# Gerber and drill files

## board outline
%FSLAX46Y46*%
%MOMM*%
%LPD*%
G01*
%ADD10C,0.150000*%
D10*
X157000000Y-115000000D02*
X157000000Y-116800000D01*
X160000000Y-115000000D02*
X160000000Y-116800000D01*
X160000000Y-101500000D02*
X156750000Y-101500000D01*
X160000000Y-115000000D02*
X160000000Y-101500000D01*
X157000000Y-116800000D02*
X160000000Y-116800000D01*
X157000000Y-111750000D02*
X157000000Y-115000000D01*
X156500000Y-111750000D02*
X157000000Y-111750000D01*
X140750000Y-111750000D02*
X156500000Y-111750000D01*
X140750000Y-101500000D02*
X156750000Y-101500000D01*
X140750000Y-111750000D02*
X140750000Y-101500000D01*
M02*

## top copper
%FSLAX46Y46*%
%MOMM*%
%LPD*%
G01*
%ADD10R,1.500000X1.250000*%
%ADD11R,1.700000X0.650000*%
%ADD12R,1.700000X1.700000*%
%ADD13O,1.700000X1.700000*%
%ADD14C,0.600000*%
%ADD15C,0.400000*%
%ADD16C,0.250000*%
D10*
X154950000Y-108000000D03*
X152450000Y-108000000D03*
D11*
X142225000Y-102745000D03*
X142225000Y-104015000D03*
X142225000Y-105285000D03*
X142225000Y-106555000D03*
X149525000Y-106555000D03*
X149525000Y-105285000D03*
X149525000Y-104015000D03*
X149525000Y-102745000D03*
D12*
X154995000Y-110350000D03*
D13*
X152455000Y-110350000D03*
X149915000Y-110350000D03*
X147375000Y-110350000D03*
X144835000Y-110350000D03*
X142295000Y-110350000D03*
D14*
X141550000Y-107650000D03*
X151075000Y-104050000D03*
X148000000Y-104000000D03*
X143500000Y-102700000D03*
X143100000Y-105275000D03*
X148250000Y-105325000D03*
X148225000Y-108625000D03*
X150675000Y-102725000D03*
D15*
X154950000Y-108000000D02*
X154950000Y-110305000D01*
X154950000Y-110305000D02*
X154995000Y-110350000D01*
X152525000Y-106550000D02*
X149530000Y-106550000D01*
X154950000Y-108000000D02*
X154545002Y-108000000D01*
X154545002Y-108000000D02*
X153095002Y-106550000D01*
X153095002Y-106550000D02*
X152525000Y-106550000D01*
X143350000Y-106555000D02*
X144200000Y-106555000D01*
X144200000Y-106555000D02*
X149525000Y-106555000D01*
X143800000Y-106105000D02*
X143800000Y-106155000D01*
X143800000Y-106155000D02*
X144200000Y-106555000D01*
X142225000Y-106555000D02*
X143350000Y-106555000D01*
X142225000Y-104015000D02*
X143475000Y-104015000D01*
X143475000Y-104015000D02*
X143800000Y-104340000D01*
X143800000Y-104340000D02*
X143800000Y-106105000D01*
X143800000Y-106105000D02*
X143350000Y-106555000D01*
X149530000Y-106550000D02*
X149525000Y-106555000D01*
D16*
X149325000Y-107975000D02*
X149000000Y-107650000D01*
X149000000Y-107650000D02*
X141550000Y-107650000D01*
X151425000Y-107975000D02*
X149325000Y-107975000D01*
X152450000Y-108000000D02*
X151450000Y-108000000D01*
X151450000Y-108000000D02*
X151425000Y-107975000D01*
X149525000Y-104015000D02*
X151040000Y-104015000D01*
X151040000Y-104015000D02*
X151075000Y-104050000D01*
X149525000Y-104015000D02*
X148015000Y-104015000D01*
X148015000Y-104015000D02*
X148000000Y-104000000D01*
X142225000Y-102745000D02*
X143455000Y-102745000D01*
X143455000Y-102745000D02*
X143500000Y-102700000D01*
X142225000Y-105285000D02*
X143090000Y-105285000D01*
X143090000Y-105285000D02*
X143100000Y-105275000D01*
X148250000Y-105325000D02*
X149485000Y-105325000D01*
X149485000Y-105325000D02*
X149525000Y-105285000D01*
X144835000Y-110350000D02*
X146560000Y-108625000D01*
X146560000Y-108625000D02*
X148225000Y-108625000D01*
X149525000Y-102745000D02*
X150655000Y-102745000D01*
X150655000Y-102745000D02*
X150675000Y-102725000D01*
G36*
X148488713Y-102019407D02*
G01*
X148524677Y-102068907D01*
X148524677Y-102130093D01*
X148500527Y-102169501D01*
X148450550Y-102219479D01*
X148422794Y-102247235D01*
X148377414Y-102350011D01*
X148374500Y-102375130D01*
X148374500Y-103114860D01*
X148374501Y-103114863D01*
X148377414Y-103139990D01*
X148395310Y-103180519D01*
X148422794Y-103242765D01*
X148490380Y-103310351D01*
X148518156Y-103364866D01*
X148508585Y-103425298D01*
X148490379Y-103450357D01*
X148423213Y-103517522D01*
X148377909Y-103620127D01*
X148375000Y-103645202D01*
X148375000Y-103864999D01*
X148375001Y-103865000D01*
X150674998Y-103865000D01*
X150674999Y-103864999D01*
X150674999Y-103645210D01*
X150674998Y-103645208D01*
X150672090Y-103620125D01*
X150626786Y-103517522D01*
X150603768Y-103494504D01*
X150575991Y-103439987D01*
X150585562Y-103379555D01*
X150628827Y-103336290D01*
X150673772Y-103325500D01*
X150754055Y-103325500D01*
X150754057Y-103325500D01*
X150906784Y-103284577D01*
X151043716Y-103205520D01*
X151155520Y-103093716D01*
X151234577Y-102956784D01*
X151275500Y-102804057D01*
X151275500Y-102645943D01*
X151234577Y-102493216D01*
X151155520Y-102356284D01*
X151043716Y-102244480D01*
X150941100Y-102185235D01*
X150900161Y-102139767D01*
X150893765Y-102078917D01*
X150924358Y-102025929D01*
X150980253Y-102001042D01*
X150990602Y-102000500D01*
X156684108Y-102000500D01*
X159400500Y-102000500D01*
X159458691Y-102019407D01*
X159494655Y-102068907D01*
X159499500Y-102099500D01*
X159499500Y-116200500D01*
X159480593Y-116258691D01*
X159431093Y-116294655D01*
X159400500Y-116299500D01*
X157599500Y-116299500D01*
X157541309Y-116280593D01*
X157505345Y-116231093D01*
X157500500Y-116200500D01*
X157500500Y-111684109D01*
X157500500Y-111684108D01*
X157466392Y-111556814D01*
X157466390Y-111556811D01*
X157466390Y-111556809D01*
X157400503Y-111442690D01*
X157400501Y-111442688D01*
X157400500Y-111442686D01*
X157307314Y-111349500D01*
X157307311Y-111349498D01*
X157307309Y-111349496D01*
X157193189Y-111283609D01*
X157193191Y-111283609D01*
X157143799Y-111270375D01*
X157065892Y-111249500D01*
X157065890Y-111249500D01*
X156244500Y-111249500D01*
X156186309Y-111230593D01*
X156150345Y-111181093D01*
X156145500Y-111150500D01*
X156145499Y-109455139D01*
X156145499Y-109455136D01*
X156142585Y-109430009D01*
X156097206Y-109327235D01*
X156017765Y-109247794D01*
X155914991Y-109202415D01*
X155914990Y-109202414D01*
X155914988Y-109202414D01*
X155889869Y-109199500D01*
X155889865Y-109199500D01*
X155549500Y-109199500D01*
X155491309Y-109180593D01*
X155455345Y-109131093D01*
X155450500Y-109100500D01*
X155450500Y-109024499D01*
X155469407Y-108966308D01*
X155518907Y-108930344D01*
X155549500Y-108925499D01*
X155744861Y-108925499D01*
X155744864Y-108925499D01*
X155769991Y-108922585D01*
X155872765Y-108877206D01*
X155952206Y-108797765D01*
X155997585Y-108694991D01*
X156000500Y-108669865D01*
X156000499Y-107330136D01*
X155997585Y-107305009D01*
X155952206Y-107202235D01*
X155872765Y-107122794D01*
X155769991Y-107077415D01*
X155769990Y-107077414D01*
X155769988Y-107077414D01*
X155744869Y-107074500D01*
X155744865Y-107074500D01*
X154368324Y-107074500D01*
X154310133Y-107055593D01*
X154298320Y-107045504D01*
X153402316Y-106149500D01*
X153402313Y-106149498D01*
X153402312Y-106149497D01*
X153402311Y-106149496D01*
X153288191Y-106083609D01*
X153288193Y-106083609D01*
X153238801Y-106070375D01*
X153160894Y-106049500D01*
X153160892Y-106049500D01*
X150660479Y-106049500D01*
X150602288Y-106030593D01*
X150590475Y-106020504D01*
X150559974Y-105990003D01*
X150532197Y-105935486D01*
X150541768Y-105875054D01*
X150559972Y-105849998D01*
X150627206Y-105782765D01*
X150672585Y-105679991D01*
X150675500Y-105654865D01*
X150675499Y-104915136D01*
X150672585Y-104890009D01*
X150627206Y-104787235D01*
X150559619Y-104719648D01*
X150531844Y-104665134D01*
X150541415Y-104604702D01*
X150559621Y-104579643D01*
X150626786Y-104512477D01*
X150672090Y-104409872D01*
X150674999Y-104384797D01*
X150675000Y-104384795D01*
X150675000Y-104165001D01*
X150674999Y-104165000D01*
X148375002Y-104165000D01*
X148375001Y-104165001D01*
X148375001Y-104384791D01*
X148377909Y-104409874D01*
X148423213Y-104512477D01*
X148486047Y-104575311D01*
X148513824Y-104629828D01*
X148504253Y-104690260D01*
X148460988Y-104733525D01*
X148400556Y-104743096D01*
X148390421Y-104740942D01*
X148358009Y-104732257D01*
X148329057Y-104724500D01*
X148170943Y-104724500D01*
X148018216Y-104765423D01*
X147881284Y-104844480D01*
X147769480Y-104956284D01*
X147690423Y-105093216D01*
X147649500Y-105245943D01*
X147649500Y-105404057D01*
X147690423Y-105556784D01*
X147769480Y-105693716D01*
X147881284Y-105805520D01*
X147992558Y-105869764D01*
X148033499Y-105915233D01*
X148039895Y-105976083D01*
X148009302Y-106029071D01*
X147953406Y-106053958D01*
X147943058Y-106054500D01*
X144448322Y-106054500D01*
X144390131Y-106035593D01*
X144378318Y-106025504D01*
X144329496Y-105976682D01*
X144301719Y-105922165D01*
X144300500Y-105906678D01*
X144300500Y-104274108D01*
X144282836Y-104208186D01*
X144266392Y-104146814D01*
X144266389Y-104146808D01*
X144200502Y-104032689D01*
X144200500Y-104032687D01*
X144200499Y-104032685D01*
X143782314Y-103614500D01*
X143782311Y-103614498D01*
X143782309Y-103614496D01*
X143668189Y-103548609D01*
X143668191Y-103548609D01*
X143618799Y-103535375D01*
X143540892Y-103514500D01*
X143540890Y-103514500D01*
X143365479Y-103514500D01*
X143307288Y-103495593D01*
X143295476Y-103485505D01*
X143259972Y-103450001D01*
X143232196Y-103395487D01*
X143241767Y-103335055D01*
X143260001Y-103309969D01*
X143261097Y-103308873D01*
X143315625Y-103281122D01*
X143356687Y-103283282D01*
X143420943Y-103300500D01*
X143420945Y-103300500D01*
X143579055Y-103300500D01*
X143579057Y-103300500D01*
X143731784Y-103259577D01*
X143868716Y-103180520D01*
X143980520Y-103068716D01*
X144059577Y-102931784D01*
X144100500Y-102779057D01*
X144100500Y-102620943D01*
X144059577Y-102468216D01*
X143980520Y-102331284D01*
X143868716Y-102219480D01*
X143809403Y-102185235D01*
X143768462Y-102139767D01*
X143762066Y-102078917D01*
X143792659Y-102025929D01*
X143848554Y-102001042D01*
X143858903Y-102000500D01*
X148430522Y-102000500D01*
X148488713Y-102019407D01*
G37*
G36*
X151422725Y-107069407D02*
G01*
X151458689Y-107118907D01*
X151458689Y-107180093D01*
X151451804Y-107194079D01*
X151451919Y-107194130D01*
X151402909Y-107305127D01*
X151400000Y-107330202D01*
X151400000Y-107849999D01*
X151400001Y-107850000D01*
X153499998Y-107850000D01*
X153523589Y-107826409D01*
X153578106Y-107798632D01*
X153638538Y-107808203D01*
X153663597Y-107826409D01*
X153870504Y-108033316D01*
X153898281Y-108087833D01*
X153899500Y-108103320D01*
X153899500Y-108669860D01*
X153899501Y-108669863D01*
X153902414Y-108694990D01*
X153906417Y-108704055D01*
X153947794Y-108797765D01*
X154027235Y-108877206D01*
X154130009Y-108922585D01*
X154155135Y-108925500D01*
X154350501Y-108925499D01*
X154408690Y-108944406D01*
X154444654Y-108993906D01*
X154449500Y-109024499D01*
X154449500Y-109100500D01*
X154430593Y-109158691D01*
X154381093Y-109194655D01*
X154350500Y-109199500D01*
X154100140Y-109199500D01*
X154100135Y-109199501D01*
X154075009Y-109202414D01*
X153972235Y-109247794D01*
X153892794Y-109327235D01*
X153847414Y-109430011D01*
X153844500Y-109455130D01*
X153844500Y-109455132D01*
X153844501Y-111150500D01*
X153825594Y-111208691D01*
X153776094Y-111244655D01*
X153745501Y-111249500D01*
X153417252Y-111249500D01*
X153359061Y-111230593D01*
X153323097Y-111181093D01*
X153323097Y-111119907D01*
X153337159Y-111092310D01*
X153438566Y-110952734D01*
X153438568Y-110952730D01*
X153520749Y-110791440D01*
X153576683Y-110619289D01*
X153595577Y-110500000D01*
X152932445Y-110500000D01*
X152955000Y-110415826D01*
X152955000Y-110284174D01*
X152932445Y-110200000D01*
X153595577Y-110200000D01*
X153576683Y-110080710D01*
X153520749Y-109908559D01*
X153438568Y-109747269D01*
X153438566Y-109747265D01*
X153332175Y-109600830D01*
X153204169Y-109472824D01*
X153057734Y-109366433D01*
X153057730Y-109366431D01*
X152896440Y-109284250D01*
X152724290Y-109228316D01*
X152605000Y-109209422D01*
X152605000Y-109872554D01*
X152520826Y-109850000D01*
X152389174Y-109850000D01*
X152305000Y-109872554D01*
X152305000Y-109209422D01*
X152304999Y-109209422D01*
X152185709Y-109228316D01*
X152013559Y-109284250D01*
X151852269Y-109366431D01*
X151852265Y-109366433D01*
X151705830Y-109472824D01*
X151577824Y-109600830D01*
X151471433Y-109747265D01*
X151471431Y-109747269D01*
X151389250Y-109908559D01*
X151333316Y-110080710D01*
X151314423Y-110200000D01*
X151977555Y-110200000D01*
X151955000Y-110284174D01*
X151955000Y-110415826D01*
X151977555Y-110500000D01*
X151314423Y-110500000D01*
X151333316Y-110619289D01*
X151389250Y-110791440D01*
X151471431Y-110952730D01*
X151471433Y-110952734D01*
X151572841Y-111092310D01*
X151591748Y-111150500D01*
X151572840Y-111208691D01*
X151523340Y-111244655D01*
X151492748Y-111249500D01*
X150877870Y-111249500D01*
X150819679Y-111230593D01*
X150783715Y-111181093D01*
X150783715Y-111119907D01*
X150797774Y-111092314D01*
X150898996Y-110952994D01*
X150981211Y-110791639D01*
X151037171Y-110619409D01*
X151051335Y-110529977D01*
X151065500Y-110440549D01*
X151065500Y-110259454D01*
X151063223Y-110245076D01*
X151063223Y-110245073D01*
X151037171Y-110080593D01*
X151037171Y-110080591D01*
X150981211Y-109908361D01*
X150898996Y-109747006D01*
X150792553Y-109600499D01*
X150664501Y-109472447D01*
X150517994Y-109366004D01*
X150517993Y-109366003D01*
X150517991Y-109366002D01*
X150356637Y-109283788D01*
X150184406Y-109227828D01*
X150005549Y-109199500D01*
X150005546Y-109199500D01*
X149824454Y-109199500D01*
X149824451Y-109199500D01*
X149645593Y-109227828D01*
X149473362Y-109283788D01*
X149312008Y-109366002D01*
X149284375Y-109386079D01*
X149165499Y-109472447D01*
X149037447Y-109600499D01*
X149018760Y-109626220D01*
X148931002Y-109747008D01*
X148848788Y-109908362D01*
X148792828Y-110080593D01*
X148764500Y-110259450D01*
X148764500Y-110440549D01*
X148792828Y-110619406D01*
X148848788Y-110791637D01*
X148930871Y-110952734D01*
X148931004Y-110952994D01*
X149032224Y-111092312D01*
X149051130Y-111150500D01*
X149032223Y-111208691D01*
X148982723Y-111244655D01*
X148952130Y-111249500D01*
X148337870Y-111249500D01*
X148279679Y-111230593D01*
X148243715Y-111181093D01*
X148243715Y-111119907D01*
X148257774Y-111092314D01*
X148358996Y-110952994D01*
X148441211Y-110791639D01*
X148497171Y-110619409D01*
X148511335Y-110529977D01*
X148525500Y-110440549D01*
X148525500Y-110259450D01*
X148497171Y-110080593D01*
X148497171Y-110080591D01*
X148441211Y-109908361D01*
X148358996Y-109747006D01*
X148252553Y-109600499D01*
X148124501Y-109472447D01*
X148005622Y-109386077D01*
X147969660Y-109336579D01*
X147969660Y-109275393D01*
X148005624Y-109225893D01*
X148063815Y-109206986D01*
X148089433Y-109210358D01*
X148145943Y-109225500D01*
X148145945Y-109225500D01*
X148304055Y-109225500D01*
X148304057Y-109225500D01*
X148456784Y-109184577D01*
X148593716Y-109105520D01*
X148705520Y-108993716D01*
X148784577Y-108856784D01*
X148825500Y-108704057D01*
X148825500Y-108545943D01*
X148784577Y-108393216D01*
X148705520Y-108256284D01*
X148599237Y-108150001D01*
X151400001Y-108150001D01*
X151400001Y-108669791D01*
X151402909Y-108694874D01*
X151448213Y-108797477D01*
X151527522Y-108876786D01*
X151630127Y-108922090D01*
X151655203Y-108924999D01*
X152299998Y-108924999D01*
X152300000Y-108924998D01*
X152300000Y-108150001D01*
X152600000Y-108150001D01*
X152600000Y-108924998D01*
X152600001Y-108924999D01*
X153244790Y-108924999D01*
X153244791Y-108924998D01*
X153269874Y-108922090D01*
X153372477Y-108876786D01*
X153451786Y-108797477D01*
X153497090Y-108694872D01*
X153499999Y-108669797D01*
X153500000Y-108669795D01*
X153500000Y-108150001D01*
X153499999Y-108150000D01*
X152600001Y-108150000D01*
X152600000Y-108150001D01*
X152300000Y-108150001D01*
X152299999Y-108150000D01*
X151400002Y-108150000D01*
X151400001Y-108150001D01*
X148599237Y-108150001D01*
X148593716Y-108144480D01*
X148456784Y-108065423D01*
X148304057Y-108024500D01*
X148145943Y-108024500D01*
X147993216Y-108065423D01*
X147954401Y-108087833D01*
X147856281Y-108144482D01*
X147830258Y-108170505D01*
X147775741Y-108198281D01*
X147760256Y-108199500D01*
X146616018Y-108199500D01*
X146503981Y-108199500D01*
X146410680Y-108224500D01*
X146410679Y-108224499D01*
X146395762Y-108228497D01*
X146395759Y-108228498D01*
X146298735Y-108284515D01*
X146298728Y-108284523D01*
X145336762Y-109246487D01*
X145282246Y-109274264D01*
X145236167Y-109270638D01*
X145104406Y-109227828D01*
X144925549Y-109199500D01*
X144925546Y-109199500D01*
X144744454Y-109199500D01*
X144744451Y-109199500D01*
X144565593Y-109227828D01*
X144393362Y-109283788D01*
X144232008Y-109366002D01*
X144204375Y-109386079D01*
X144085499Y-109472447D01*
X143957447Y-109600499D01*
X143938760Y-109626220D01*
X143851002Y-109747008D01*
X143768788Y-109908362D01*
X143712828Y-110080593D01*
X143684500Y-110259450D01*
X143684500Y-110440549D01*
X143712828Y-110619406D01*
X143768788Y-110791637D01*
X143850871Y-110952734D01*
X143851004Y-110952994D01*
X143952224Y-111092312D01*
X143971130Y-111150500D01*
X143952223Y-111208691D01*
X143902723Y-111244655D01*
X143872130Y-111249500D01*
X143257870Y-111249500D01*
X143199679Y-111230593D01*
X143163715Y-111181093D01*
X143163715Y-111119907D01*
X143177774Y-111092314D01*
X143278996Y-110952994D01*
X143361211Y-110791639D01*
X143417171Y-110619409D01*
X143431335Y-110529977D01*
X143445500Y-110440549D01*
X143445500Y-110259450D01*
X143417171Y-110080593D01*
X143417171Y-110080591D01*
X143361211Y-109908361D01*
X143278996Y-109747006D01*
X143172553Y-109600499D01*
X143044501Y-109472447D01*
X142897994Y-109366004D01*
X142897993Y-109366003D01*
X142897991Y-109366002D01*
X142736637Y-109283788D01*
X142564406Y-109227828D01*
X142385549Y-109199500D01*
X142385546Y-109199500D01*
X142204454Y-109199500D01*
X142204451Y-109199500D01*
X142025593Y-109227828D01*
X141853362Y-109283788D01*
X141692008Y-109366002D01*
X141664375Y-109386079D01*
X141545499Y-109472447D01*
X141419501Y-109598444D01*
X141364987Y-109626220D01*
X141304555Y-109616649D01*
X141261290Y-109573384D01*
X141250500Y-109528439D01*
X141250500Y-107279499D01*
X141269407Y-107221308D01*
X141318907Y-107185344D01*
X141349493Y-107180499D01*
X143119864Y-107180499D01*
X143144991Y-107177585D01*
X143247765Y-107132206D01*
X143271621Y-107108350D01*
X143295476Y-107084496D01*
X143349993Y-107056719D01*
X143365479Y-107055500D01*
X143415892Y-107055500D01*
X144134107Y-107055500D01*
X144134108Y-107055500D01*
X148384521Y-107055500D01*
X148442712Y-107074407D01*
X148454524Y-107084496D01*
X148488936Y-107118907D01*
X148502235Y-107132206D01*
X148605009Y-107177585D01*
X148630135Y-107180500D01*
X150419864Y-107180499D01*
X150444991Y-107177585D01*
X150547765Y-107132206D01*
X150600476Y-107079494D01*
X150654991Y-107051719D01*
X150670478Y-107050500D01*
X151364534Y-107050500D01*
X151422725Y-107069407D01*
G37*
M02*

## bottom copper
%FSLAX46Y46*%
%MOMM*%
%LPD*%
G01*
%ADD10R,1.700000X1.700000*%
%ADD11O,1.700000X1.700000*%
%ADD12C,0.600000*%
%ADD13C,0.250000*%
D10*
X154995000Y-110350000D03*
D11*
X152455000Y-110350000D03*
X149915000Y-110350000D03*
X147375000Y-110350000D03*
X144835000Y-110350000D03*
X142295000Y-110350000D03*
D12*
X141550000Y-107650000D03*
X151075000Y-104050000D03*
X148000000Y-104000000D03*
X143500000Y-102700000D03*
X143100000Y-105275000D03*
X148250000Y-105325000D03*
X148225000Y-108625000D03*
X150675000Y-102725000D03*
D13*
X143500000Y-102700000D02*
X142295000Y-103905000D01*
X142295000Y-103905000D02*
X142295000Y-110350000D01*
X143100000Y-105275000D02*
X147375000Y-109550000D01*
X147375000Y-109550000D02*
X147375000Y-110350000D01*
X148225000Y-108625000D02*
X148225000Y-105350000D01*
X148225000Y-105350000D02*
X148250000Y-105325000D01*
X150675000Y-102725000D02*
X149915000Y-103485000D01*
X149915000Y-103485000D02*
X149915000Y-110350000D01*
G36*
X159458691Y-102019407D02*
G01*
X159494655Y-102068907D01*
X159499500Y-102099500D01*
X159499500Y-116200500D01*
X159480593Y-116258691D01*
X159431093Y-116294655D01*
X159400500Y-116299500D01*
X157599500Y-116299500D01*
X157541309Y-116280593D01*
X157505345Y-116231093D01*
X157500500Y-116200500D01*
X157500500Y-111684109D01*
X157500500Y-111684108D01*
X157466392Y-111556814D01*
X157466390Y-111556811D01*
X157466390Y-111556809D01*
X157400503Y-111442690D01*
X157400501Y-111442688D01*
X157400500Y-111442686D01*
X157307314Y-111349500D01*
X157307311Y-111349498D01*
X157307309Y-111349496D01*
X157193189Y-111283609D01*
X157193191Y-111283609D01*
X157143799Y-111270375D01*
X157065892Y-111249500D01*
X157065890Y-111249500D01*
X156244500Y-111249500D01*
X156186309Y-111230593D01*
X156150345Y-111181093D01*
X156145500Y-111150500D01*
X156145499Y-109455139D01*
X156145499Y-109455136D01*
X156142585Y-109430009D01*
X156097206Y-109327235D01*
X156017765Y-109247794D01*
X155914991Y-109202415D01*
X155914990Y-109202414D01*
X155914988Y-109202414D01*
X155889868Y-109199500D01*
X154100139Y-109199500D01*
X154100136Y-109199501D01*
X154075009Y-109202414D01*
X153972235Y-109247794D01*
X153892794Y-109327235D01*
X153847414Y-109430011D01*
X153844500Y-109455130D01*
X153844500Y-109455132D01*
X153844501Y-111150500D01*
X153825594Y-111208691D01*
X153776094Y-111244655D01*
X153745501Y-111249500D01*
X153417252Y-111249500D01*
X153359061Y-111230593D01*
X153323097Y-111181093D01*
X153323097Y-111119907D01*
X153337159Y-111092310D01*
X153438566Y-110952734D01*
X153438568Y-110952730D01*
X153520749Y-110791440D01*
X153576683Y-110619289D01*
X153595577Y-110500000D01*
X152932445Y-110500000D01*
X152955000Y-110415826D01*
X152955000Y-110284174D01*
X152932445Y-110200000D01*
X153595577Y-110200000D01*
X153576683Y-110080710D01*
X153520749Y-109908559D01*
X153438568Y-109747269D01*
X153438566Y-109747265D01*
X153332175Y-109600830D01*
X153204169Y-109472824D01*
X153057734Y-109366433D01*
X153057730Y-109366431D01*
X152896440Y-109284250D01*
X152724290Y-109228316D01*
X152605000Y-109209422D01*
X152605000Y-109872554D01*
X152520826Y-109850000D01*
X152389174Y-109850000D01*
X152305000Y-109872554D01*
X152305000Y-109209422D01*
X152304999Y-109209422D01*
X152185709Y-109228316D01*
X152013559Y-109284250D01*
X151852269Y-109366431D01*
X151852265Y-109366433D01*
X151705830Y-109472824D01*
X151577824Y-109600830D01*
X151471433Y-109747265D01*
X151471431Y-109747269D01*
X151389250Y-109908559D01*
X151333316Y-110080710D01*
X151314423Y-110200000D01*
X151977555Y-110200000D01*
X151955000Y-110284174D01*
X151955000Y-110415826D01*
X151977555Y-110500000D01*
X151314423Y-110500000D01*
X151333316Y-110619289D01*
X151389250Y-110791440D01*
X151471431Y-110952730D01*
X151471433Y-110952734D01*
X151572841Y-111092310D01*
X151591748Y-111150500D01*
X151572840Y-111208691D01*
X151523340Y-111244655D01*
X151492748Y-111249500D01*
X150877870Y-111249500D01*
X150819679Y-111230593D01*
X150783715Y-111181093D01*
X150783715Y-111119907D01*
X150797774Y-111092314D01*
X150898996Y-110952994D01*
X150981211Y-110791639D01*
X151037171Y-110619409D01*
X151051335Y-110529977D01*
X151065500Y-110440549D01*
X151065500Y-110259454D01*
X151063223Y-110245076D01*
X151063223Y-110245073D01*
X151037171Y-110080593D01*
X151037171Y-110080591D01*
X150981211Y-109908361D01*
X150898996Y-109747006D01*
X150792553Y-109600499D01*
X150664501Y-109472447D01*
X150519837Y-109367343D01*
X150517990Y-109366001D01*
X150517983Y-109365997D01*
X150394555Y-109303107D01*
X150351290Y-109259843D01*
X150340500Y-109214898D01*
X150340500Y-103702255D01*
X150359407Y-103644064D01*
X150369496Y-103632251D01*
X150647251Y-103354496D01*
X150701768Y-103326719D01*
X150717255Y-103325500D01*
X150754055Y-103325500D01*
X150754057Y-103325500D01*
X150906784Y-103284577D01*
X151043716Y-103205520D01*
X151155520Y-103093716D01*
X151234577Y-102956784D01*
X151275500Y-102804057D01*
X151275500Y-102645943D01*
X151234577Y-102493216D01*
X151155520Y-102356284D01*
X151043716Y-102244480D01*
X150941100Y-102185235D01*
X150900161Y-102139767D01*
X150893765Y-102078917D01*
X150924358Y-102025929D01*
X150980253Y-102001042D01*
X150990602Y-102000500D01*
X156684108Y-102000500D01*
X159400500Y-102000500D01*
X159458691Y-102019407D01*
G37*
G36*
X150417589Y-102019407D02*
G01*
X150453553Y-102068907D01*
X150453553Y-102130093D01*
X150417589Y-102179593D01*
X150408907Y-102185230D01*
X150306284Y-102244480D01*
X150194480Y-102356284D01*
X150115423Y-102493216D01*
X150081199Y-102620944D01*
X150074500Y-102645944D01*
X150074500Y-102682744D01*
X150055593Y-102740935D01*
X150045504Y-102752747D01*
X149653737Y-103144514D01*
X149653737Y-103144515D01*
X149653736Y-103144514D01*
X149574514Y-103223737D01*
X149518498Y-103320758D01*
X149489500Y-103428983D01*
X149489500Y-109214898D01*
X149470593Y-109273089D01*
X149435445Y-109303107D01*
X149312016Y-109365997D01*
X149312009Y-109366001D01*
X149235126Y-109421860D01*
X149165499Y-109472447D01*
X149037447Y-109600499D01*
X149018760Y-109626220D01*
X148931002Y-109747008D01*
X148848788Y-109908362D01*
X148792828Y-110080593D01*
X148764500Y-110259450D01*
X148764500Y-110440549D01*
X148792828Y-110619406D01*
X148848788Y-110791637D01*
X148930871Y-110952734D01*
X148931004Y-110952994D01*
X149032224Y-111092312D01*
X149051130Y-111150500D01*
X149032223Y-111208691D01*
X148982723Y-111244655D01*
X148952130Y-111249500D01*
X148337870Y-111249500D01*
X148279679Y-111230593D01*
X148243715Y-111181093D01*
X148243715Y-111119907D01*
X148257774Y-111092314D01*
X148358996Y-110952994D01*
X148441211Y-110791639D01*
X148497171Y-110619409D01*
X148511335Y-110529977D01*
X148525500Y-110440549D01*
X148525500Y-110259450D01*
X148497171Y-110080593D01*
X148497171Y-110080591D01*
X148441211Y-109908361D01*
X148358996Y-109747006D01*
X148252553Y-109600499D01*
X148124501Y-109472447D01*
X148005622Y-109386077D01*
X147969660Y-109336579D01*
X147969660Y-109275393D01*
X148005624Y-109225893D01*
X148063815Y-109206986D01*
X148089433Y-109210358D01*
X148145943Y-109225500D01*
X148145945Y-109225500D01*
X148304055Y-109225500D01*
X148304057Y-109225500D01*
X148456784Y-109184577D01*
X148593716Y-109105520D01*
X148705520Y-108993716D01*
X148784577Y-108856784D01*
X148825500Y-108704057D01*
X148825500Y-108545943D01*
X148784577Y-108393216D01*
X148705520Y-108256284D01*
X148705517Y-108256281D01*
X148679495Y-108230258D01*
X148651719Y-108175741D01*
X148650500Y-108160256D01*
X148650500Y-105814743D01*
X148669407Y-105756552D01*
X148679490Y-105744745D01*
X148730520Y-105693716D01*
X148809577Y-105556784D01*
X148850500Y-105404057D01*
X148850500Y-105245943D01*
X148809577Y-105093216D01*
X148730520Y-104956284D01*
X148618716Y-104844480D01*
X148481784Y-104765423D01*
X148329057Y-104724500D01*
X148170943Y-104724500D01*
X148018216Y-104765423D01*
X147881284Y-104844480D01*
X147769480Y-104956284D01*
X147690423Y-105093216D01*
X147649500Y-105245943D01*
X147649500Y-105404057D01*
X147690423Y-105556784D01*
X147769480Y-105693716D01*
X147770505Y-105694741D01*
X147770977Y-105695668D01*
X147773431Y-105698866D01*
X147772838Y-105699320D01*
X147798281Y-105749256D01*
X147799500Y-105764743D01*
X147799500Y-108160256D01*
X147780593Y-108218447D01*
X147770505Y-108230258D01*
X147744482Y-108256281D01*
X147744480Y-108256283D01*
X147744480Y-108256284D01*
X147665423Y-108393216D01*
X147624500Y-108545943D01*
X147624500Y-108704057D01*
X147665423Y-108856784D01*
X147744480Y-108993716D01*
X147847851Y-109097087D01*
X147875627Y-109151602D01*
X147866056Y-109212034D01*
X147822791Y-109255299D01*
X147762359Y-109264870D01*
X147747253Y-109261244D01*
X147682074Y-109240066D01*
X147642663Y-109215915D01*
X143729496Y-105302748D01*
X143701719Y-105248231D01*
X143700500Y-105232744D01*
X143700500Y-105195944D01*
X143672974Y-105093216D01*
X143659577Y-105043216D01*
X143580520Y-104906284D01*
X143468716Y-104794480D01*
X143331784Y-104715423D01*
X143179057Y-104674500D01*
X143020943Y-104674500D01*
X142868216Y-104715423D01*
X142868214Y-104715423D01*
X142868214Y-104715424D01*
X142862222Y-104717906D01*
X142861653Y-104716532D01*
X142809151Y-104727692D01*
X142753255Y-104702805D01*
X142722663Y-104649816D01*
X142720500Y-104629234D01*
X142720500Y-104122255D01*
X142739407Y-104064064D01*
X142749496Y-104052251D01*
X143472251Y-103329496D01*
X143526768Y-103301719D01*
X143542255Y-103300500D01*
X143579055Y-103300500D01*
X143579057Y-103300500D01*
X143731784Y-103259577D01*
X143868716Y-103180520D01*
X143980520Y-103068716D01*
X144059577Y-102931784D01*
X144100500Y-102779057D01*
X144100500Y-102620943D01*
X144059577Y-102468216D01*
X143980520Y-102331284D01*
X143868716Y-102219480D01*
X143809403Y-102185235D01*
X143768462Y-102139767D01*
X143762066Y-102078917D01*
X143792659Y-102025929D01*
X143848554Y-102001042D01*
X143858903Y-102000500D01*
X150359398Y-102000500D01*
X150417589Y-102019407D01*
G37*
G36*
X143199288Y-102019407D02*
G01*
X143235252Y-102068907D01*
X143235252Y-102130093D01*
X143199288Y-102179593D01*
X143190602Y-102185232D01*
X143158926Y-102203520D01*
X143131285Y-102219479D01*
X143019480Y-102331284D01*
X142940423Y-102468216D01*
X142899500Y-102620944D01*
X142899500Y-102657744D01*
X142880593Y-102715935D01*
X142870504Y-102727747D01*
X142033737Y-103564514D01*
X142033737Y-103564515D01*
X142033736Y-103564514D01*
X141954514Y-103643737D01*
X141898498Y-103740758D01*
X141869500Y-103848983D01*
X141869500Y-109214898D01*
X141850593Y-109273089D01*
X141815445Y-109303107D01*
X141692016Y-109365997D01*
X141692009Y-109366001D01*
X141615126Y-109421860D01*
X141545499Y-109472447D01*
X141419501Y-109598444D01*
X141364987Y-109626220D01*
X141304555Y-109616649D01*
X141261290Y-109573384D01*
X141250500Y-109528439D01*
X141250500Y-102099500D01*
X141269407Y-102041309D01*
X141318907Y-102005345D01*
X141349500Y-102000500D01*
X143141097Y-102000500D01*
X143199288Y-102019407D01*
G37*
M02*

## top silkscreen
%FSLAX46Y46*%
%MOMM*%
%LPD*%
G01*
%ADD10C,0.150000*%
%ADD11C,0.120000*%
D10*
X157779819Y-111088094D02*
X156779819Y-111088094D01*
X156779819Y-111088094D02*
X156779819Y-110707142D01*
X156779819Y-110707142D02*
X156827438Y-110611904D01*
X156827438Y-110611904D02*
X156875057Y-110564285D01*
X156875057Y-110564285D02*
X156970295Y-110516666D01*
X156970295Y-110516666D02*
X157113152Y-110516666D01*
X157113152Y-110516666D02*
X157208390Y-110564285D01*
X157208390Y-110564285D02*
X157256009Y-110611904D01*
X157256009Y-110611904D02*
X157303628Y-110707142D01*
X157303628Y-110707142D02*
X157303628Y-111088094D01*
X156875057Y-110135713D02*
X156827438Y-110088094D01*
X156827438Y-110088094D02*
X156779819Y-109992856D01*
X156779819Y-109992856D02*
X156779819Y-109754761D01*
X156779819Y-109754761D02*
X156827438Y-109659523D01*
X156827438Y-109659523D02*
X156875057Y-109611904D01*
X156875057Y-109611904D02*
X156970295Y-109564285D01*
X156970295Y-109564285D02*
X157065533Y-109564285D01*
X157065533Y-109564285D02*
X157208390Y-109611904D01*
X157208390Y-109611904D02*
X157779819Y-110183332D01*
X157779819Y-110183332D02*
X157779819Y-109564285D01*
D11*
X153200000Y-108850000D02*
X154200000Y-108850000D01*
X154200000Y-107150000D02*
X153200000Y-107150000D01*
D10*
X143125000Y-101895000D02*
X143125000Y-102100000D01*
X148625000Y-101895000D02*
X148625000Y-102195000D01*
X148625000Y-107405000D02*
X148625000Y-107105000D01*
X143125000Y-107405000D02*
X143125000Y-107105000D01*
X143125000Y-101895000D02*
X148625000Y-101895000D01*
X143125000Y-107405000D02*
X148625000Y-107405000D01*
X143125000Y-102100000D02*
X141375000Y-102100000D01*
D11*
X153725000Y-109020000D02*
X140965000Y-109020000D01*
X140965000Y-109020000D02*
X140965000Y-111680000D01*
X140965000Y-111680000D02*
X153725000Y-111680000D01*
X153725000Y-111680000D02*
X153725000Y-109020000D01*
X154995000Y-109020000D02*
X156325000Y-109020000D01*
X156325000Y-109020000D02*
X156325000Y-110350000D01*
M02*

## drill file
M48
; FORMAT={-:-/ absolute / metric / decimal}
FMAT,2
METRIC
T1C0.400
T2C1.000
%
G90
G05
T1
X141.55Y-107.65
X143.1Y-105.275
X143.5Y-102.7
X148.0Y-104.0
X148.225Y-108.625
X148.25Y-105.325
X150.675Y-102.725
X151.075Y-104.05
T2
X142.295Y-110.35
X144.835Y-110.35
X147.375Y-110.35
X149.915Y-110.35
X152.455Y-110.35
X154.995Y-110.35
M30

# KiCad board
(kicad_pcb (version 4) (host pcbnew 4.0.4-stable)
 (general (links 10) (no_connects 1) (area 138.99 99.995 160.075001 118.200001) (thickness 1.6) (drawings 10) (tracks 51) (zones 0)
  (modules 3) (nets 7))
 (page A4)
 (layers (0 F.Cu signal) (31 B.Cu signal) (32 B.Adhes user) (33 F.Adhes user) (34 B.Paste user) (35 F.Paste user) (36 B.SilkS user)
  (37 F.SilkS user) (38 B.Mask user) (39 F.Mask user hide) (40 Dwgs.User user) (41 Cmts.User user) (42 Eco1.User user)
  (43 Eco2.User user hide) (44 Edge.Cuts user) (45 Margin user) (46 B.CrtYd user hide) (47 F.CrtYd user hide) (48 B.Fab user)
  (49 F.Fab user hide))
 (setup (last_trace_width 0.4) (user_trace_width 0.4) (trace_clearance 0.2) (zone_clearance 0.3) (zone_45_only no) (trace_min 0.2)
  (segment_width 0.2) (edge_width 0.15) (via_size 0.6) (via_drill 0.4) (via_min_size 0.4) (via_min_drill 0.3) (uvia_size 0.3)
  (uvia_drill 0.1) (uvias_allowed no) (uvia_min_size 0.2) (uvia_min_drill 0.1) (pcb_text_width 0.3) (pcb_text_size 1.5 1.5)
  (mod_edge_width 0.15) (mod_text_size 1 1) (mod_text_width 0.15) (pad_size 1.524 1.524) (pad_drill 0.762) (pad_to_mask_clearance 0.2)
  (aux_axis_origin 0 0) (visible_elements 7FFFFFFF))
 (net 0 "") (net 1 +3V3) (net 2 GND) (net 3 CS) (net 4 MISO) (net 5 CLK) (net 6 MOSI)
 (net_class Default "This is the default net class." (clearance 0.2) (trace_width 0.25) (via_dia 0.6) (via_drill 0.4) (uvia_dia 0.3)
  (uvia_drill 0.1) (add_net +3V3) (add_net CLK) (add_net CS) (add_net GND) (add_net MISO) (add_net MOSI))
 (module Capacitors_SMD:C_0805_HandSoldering (layer F.Cu) (at 153.7 108 180)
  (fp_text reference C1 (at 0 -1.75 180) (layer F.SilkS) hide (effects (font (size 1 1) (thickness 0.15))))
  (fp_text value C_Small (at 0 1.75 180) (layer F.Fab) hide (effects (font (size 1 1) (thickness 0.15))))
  (fp_line (start 0.5 -0.85) (end -0.5 -0.85) (layer F.SilkS) (width 0.12))
  (fp_line (start -0.5 0.85) (end 0.5 0.85) (layer F.SilkS) (width 0.12))
  (pad 1 smd rect (at -1.25 0 180) (size 1.5 1.25) (layers F.Cu F.Paste F.Mask) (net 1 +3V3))
  (pad 2 smd rect (at 1.25 0 180) (size 1.5 1.25) (layers F.Cu F.Paste F.Mask) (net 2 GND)))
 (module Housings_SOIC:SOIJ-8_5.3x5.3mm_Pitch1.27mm (layer F.Cu) (at 145.875 104.65)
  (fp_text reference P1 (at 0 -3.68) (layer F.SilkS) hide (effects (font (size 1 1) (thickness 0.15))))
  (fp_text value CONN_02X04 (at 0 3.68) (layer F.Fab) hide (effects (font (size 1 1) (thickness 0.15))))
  (fp_line (start -2.75 -2.755) (end -2.75 -2.55) (layer F.SilkS) (width 0.15))
  (fp_line (start 2.75 -2.755) (end 2.75 -2.455) (layer F.SilkS) (width 0.15))
  (fp_line (start 2.75 2.755) (end 2.75 2.455) (layer F.SilkS) (width 0.15))
  (fp_line (start -2.75 2.755) (end -2.75 2.455) (layer F.SilkS) (width 0.15))
  (fp_line (start -2.75 -2.755) (end 2.75 -2.755) (layer F.SilkS) (width 0.15))
  (fp_line (start -2.75 2.755) (end 2.75 2.755) (layer F.SilkS) (width 0.15))
  (fp_line (start -2.75 -2.55) (end -4.5 -2.55) (layer F.SilkS) (width 0.15))
  (pad 1 smd rect (at -3.65 -1.905) (size 1.7 0.65) (layers F.Cu F.Paste F.Mask) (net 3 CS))
  (pad 2 smd rect (at -3.65 -0.635) (size 1.7 0.65) (layers F.Cu F.Paste F.Mask) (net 1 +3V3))
  (pad 3 smd rect (at -3.65 0.635) (size 1.7 0.65) (layers F.Cu F.Paste F.Mask) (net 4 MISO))
  (pad 4 smd rect (at -3.65 1.905) (size 1.7 0.65) (layers F.Cu F.Paste F.Mask) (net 1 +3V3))
  (pad 5 smd rect (at 3.65 1.905) (size 1.7 0.65) (layers F.Cu F.Paste F.Mask) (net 1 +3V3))
  (pad 6 smd rect (at 3.65 0.635) (size 1.7 0.65) (layers F.Cu F.Paste F.Mask) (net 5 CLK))
  (pad 7 smd rect (at 3.65 -0.635) (size 1.7 0.65) (layers F.Cu F.Paste F.Mask) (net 2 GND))
  (pad 8 smd rect (at 3.65 -1.905) (size 1.7 0.65) (layers F.Cu F.Paste F.Mask) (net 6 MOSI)))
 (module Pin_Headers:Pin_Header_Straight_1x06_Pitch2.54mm (layer F.Cu) (at 154.995 110.35 270)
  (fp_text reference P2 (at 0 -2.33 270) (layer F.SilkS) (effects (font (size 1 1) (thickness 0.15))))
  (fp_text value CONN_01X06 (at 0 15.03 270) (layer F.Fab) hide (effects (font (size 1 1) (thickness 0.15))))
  (fp_line (start -1.33 1.27) (end -1.33 14.03) (layer F.SilkS) (width 0.12))
  (fp_line (start -1.33 14.03) (end 1.33 14.03) (layer F.SilkS) (width 0.12))
  (fp_line (start 1.33 14.03) (end 1.33 1.27) (layer F.SilkS) (width 0.12))
  (fp_line (start 1.33 1.27) (end -1.33 1.27) (layer F.SilkS) (width 0.12))
  (fp_line (start -1.33 0) (end -1.33 -1.33) (layer F.SilkS) (width 0.12))
  (fp_line (start -1.33 -1.33) (end 0 -1.33) (layer F.SilkS) (width 0.12))
  (pad 1 thru_hole rect (at 0 0 270) (size 1.7 1.7) (drill 1) (layers *.Cu *.Mask) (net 1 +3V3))
  (pad 2 thru_hole oval (at 0 2.54 270) (size 1.7 1.7) (drill 1) (layers *.Cu *.Mask) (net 2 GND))
  (pad 3 thru_hole oval (at 0 5.08 270) (size 1.7 1.7) (drill 1) (layers *.Cu *.Mask) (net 6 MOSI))
  (pad 4 thru_hole oval (at 0 7.62 270) (size 1.7 1.7) (drill 1) (layers *.Cu *.Mask) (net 4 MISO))
  (pad 5 thru_hole oval (at 0 10.16 270) (size 1.7 1.7) (drill 1) (layers *.Cu *.Mask) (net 5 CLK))
  (pad 6 thru_hole oval (at 0 12.7 270) (size 1.7 1.7) (drill 1) (layers *.Cu *.Mask) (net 3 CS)))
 (gr_line (start 157 115) (end 157 116.8) (layer Edge.Cuts) (width 0.15))
 (gr_line (start 160 115) (end 160 116.8) (layer Edge.Cuts) (width 0.15))
 (gr_line (start 160 101.5) (end 156.75 101.5) (layer Edge.Cuts) (width 0.15))
 (gr_line (start 160 115) (end 160 101.5) (layer Edge.Cuts) (width 0.15))
 (gr_line (start 157 116.8) (end 160 116.8) (layer Edge.Cuts) (width 0.15))
 (gr_line (start 157 111.75) (end 157 115) (layer Edge.Cuts) (width 0.15))
 (gr_line (start 156.5 111.75) (end 157 111.75) (layer Edge.Cuts) (width 0.15))
 (gr_line (start 140.75 111.75) (end 156.5 111.75) (layer Edge.Cuts) (width 0.15))
 (gr_line (start 140.75 101.5) (end 156.75 101.5) (layer Edge.Cuts) (width 0.15))
 (gr_line (start 140.75 111.75) (end 140.75 101.5) (layer Edge.Cuts) (width 0.15))
 (segment (start 154.95 108) (end 154.95 110.305) (width 0.4) (layer F.Cu) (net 1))
 (segment (start 154.95 110.305) (end 154.995 110.35) (width 0.4) (layer F.Cu) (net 1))
 (segment (start 152.525 106.55) (end 149.53 106.55) (width 0.4) (layer F.Cu) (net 1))
 (segment (start 154.95 108) (end 154.545002 108) (width 0.4) (layer F.Cu) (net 1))
 (segment (start 154.545002 108) (end 153.095002 106.55) (width 0.4) (layer F.Cu) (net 1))
 (segment (start 153.095002 106.55) (end 152.525 106.55) (width 0.4) (layer F.Cu) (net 1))
 (segment (start 143.35 106.555) (end 144.2 106.555) (width 0.4) (layer F.Cu) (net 1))
 (segment (start 144.2 106.555) (end 149.525 106.555) (width 0.4) (layer F.Cu) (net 1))
 (segment (start 143.8 106.105) (end 143.8 106.155) (width 0.4) (layer F.Cu) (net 1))
 (segment (start 143.8 106.155) (end 144.2 106.555) (width 0.4) (layer F.Cu) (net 1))
 (segment (start 142.225 106.555) (end 143.35 106.555) (width 0.4) (layer F.Cu) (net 1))
 (segment (start 142.225 104.015) (end 143.475 104.015) (width 0.4) (layer F.Cu) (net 1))
 (segment (start 143.475 104.015) (end 143.8 104.34) (width 0.4) (layer F.Cu) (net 1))
 (segment (start 143.8 104.34) (end 143.8 106.105) (width 0.4) (layer F.Cu) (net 1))
 (segment (start 143.8 106.105) (end 143.35 106.555) (width 0.4) (layer F.Cu) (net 1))
 (segment (start 149.53 106.55) (end 149.525 106.555) (width 0.4) (layer F.Cu) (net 1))
 (segment (start 149.325 107.975) (end 149 107.65) (width 0.25) (layer F.Cu) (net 2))
 (segment (start 149 107.65) (end 141.55 107.65) (width 0.25) (layer F.Cu) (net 2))
 (via (at 141.55 107.65) (size 0.6) (drill 0.4) (layers F.Cu B.Cu) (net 2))
 (segment (start 151.425 107.975) (end 149.325 107.975) (width 0.25) (layer F.Cu) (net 2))
 (segment (start 152.45 108) (end 151.45 108) (width 0.25) (layer F.Cu) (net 2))
 (segment (start 151.45 108) (end 151.425 107.975) (width 0.25) (layer F.Cu) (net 2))
 (segment (start 149.525 104.015) (end 151.04 104.015) (width 0.25) (layer F.Cu) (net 2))
 (segment (start 151.04 104.015) (end 151.075 104.05) (width 0.25) (layer F.Cu) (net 2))
 (via (at 151.075 104.05) (size 0.6) (drill 0.4) (layers F.Cu B.Cu) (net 2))
 (segment (start 149.525 104.015) (end 148.015 104.015) (width 0.25) (layer F.Cu) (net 2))
 (segment (start 148.015 104.015) (end 148 104) (width 0.25) (layer F.Cu) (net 2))
 (via (at 148 104) (size 0.6) (drill 0.4) (layers F.Cu B.Cu) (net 2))
 (segment (start 143.5 102.7) (end 142.295 103.905) (width 0.25) (layer B.Cu) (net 3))
 (segment (start 142.295 103.905) (end 142.295 110.35) (width 0.25) (layer B.Cu) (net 3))
 (segment (start 142.225 102.745) (end 143.455 102.745) (width 0.25) (layer F.Cu) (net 3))
 (segment (start 143.455 102.745) (end 143.5 102.7) (width 0.25) (layer F.Cu) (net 3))
 (via (at 143.5 102.7) (size 0.6) (drill 0.4) (layers F.Cu B.Cu) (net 3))
 (segment (start 143.1 105.275) (end 147.375 109.55) (width 0.25) (layer B.Cu) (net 4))
 (segment (start 147.375 109.55) (end 147.375 110.35) (width 0.25) (layer B.Cu) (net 4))
 (segment (start 142.225 105.285) (end 143.09 105.285) (width 0.25) (layer F.Cu) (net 4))
 (segment (start 143.09 105.285) (end 143.1 105.275) (width 0.25) (layer F.Cu) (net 4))
 (via (at 143.1 105.275) (size 0.6) (drill 0.4) (layers F.Cu B.Cu) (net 4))
 (segment (start 148.25 105.325) (end 149.485 105.325) (width 0.25) (layer F.Cu) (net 5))
 (segment (start 149.485 105.325) (end 149.525 105.285) (width 0.25) (layer F.Cu) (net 5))
 (segment (start 148.225 108.625) (end 148.225 105.35) (width 0.25) (layer B.Cu) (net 5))
 (segment (start 148.225 105.35) (end 148.25 105.325) (width 0.25) (layer B.Cu) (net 5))
 (via (at 148.25 105.325) (size 0.6) (drill 0.4) (layers F.Cu B.Cu) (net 5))
 (segment (start 144.835 110.35) (end 146.56 108.625) (width 0.25) (layer F.Cu) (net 5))
 (segment (start 146.56 108.625) (end 148.225 108.625) (width 0.25) (layer F.Cu) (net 5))
 (via (at 148.225 108.625) (size 0.6) (drill 0.4) (layers F.Cu B.Cu) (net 5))
 (segment (start 150.675 102.725) (end 149.915 103.485) (width 0.25) (layer B.Cu) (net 6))
 (segment (start 149.915 103.485) (end 149.915 110.35) (width 0.25) (layer B.Cu) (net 6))
 (segment (start 149.525 102.745) (end 150.655 102.745) (width 0.25) (layer F.Cu) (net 6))
 (segment (start 150.655 102.745) (end 150.675 102.725) (width 0.25) (layer F.Cu) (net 6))
 (via (at 150.675 102.725) (size 0.6) (drill 0.4) (layers F.Cu B.Cu) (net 6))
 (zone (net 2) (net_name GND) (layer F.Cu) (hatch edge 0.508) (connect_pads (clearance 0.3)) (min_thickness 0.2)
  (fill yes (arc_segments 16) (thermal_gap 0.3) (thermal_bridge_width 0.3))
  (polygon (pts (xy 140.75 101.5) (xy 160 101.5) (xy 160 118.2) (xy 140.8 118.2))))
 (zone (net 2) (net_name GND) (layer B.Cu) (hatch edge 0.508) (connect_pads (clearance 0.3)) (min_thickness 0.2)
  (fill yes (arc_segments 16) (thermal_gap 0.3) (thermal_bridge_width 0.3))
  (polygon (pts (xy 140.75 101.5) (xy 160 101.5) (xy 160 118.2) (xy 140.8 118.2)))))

